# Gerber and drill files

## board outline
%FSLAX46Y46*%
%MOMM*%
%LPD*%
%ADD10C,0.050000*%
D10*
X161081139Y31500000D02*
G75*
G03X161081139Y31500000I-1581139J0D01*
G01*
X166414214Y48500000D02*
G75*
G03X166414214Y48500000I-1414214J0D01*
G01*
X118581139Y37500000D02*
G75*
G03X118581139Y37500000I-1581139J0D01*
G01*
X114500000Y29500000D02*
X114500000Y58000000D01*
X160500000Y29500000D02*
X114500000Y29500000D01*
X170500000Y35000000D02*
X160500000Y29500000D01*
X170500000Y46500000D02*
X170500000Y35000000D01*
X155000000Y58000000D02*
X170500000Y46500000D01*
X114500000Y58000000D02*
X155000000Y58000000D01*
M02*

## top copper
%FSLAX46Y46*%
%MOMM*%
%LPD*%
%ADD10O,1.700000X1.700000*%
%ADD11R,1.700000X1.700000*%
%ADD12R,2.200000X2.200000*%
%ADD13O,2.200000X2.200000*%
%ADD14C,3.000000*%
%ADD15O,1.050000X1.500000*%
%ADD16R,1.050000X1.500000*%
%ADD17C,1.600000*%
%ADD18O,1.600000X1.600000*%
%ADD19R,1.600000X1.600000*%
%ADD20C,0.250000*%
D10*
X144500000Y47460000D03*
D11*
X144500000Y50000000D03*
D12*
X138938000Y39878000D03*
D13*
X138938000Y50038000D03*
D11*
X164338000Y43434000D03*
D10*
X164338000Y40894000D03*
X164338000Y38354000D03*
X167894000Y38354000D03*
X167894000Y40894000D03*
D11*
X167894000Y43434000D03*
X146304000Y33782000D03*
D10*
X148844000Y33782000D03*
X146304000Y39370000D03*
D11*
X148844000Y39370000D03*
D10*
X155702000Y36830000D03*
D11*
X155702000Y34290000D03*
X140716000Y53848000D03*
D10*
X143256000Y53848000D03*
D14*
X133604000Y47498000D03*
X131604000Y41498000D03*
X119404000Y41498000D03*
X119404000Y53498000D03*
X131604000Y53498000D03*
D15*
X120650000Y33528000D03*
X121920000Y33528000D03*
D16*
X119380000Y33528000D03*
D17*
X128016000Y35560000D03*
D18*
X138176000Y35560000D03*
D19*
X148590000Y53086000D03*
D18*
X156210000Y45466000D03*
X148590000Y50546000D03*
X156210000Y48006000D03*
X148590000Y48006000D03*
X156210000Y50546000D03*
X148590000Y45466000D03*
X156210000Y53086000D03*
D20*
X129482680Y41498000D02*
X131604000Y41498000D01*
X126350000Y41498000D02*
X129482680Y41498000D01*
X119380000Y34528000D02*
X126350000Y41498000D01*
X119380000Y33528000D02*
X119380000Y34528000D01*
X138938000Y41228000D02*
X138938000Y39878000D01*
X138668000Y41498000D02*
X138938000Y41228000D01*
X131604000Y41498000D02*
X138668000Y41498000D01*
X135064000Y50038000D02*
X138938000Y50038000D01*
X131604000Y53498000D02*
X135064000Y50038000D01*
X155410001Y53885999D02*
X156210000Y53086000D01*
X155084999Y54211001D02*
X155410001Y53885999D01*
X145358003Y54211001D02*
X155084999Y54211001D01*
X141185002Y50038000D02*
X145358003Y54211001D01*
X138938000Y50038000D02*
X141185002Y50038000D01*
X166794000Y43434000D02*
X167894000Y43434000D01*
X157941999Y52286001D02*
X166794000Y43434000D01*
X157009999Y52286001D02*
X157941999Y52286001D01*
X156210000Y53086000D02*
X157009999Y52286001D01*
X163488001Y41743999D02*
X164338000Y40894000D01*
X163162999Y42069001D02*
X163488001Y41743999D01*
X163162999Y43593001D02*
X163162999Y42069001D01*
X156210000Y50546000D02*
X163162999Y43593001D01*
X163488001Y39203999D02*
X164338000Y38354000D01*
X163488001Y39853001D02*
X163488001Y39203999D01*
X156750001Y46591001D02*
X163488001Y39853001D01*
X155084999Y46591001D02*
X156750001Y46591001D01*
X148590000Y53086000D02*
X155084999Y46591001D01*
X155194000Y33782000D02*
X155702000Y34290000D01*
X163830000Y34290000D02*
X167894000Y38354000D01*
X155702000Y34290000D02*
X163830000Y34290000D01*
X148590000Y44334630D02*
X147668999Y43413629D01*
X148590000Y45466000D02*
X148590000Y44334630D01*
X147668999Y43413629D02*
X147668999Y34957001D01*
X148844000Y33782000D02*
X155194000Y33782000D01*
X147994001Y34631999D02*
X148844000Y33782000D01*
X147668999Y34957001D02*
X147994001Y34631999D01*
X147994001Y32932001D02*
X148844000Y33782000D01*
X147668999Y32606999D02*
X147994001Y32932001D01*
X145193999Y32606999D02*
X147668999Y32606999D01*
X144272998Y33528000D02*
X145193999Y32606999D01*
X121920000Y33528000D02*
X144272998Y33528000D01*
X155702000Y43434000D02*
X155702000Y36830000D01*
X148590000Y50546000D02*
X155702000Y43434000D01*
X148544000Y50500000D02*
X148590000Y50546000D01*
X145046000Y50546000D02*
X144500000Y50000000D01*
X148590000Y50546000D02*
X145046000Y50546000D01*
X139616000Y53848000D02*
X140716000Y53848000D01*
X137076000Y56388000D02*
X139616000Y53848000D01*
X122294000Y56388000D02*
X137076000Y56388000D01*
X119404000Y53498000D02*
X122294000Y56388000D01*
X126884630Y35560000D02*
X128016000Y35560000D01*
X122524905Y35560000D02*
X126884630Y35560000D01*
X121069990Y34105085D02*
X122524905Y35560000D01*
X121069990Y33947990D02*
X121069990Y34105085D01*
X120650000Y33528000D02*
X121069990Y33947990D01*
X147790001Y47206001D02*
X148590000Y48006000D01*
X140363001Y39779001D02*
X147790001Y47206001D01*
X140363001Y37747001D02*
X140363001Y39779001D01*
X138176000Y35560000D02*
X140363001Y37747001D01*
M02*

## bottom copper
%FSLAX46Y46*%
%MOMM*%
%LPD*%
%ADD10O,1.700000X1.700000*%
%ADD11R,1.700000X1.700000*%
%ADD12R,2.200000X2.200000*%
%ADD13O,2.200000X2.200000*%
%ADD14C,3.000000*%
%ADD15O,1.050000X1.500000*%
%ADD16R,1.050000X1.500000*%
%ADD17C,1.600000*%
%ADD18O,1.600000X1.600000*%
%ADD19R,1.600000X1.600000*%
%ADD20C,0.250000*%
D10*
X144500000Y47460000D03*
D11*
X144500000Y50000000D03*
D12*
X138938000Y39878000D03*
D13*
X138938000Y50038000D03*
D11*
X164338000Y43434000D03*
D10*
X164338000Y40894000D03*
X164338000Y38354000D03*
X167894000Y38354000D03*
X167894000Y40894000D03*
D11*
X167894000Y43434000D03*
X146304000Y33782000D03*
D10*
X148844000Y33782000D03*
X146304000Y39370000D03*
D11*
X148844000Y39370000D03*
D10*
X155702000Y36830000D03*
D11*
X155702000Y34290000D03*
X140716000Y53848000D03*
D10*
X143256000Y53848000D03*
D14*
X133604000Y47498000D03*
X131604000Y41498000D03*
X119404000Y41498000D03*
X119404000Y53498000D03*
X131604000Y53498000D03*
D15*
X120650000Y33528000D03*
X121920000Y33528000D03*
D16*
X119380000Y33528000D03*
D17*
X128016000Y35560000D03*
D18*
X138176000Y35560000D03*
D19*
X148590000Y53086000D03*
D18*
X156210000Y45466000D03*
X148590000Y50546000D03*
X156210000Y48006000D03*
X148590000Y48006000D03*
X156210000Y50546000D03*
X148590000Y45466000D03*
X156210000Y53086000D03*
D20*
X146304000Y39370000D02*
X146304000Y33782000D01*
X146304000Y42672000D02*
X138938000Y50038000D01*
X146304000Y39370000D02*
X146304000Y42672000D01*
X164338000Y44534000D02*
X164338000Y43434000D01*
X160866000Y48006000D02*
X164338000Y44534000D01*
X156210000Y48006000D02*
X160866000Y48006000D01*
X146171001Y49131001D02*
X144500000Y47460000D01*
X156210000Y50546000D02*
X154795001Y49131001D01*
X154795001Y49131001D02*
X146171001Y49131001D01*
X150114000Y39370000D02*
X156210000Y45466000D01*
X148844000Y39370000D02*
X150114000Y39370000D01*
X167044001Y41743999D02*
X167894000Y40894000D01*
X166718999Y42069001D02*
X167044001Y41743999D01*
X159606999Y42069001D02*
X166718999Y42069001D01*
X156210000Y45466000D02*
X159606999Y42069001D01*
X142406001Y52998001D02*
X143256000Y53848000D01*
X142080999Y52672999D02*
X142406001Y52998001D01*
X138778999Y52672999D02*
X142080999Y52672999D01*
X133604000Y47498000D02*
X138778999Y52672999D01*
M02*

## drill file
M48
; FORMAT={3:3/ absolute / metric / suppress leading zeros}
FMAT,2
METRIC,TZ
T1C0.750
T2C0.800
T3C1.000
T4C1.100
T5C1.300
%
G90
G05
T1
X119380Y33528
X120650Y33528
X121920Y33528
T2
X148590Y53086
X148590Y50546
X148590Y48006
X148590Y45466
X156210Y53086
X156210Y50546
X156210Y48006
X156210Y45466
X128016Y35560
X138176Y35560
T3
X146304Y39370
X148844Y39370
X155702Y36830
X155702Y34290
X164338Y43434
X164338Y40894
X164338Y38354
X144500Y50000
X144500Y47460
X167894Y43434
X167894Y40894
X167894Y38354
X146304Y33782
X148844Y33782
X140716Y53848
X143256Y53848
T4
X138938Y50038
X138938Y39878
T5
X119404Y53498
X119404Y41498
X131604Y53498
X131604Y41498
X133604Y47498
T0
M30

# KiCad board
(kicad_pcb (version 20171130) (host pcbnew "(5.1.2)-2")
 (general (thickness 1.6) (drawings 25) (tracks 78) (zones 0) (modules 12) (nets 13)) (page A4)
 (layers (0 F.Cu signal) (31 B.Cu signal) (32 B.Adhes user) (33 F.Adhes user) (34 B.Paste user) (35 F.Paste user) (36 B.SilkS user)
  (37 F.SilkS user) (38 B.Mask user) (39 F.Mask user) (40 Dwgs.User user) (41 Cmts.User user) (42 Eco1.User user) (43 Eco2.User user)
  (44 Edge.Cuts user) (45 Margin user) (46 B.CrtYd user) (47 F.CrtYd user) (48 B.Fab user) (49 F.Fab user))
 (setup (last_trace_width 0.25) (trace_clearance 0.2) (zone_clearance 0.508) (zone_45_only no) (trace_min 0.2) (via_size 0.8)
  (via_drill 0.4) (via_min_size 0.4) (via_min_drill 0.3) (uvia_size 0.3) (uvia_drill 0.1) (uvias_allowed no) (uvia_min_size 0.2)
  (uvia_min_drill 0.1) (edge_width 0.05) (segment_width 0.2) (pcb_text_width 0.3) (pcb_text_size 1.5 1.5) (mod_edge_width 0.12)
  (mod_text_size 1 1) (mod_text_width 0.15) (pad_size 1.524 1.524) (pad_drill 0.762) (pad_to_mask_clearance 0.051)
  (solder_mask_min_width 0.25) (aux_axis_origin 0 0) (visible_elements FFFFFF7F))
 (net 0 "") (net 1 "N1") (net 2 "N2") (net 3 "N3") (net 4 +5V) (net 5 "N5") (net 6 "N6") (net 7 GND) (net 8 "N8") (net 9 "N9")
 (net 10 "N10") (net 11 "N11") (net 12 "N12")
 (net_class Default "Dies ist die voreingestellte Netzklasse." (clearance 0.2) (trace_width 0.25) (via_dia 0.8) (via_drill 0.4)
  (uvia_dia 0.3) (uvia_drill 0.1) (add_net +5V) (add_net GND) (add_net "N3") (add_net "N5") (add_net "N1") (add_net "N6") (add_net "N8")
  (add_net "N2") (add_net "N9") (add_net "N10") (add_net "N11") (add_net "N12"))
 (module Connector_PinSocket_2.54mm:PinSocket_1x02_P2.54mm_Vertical (layer F.Cu) (at 144.5 -50)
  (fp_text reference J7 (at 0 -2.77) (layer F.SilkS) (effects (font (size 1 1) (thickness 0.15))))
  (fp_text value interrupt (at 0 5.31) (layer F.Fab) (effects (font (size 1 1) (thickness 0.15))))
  (pad 2 thru_hole oval (at 0 2.54) (size 1.7 1.7) (drill 1) (layers *.Cu *.Mask) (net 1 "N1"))
  (pad 1 thru_hole rect (at 0 0) (size 1.7 1.7) (drill 1) (layers *.Cu *.Mask) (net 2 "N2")))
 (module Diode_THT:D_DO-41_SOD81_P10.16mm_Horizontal (layer F.Cu) (at 138.938 -39.878 90)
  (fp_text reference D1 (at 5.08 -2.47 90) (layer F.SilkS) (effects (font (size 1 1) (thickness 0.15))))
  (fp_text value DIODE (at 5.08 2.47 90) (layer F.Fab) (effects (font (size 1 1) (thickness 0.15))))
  (pad 1 thru_hole rect (at 0 0 90) (size 2.2 2.2) (drill 1.1) (layers *.Cu *.Mask) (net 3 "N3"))
  (pad 2 thru_hole oval (at 10.16 0 90) (size 2.2 2.2) (drill 1.1) (layers *.Cu *.Mask) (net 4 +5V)))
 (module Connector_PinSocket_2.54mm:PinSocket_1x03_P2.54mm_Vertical (layer F.Cu) (at 164.338 -43.434)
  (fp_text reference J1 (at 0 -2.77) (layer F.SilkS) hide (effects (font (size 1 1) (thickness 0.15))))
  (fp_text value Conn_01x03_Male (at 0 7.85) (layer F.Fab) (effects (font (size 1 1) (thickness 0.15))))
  (pad 1 thru_hole rect (at 0 0) (size 1.7 1.7) (drill 1) (layers *.Cu *.Mask) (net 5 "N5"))
  (pad 2 thru_hole oval (at 0 2.54) (size 1.7 1.7) (drill 1) (layers *.Cu *.Mask) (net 1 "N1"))
  (pad 3 thru_hole oval (at 0 5.08) (size 1.7 1.7) (drill 1) (layers *.Cu *.Mask) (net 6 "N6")))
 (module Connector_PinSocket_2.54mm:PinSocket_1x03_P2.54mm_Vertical (layer F.Cu) (at 167.894 -43.434)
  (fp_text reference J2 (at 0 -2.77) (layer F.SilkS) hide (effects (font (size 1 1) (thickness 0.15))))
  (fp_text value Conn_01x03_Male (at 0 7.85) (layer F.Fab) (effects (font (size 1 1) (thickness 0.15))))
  (pad 3 thru_hole oval (at 0 5.08) (size 1.7 1.7) (drill 1) (layers *.Cu *.Mask) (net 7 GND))
  (pad 2 thru_hole oval (at 0 2.54) (size 1.7 1.7) (drill 1) (layers *.Cu *.Mask) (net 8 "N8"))
  (pad 1 thru_hole rect (at 0 0) (size 1.7 1.7) (drill 1) (layers *.Cu *.Mask) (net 4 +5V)))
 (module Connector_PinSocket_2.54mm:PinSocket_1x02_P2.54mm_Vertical (layer F.Cu) (at 146.304 -33.782 90)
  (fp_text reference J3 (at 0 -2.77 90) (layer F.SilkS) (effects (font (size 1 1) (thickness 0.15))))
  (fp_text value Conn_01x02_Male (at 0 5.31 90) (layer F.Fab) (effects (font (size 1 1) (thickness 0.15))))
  (pad 1 thru_hole rect (at 0 0 90) (size 1.7 1.7) (drill 1) (layers *.Cu *.Mask) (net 4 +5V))
  (pad 2 thru_hole oval (at 0 2.54 90) (size 1.7 1.7) (drill 1) (layers *.Cu *.Mask) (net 7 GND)))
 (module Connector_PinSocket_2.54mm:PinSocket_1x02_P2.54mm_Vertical (layer F.Cu) (at 148.844 -39.37 270)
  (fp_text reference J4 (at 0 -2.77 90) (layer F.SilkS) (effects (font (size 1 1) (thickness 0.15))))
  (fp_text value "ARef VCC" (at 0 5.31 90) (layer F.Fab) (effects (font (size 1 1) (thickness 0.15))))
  (pad 2 thru_hole oval (at 0 2.54 270) (size 1.7 1.7) (drill 1) (layers *.Cu *.Mask) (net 4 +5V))
  (pad 1 thru_hole rect (at 0 0 270) (size 1.7 1.7) (drill 1) (layers *.Cu *.Mask) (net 8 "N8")))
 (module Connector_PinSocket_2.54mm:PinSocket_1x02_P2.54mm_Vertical (layer F.Cu) (at 155.702 -34.29 180)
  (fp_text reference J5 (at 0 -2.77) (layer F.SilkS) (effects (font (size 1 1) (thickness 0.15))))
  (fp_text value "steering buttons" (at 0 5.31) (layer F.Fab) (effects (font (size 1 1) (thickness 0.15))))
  (pad 2 thru_hole oval (at 0 2.54 180) (size 1.7 1.7) (drill 1) (layers *.Cu *.Mask) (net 2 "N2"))
  (pad 1 thru_hole rect (at 0 0 180) (size 1.7 1.7) (drill 1) (layers *.Cu *.Mask) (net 7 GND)))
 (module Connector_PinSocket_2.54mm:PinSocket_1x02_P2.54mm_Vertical (layer F.Cu) (at 140.716 -53.848 90)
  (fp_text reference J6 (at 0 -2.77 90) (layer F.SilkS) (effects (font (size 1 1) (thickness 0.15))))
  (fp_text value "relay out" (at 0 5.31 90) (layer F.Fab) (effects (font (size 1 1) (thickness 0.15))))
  (pad 1 thru_hole rect (at 0 0 90) (size 1.7 1.7) (drill 1) (layers *.Cu *.Mask) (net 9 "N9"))
  (pad 2 thru_hole oval (at 0 2.54 90) (size 1.7 1.7) (drill 1) (layers *.Cu *.Mask) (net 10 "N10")))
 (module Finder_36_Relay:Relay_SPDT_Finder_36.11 (layer F.Cu) (at 133.604 -47.498 180)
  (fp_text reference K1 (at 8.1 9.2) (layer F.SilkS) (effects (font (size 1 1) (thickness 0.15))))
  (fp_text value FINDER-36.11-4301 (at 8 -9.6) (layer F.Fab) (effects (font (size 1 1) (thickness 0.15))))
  (pad 11 thru_hole circle (at 0 0 180) (size 3 3) (drill 1.3) (layers *.Cu *.Mask) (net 10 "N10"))
  (pad A2 thru_hole circle (at 2 -6 180) (size 3 3) (drill 1.3) (layers *.Cu *.Mask) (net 3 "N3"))
  (pad 12 thru_hole circle (at 14.2 -6 180) (size 3 3) (drill 1.3) (layers *.Cu *.Mask))
  (pad 14 thru_hole circle (at 14.2 6 180) (size 3 3) (drill 1.3) (layers *.Cu *.Mask) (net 9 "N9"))
  (pad A1 thru_hole circle (at 2 6 180) (size 3 3) (drill 1.3) (layers *.Cu *.Mask) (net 4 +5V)))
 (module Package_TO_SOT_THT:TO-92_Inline (layer F.Cu) (at 119.38 -33.528)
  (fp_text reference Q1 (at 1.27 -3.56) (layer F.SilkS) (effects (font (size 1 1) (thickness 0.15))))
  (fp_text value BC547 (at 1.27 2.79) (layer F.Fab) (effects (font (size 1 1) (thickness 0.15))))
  (pad 2 thru_hole oval (at 1.27 0) (size 1.05 1.5) (drill 0.75) (layers *.Cu *.Mask) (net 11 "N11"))
  (pad 3 thru_hole oval (at 2.54 0) (size 1.05 1.5) (drill 0.75) (layers *.Cu *.Mask) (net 7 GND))
  (pad 1 thru_hole rect (at 0 0) (size 1.05 1.5) (drill 0.75) (layers *.Cu *.Mask) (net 3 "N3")))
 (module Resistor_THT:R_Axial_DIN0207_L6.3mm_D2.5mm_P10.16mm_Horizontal (layer F.Cu) (at 128.016 -35.56)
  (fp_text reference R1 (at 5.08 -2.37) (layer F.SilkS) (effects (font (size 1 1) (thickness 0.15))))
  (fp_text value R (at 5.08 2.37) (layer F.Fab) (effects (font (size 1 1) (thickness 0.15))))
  (pad 1 thru_hole circle (at 0 0) (size 1.6 1.6) (drill 0.8) (layers *.Cu *.Mask) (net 11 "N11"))
  (pad 2 thru_hole oval (at 10.16 0) (size 1.6 1.6) (drill 0.8) (layers *.Cu *.Mask) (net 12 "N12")))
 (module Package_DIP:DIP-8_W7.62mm (layer F.Cu) (at 148.59 -53.086)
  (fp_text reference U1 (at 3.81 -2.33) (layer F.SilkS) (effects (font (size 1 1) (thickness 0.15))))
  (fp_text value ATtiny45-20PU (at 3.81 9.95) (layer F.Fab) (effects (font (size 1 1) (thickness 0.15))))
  (pad 1 thru_hole rect (at 0 0) (size 1.6 1.6) (drill 0.8) (layers *.Cu *.Mask) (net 6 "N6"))
  (pad 5 thru_hole oval (at 7.62 7.62) (size 1.6 1.6) (drill 0.8) (layers *.Cu *.Mask) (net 8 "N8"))
  (pad 2 thru_hole oval (at 0 2.54) (size 1.6 1.6) (drill 0.8) (layers *.Cu *.Mask) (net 2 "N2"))
  (pad 6 thru_hole oval (at 7.62 5.08) (size 1.6 1.6) (drill 0.8) (layers *.Cu *.Mask) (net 5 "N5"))
  (pad 3 thru_hole oval (at 0 5.08) (size 1.6 1.6) (drill 0.8) (layers *.Cu *.Mask) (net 12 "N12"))
  (pad 7 thru_hole oval (at 7.62 2.54) (size 1.6 1.6) (drill 0.8) (layers *.Cu *.Mask) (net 1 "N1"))
  (pad 4 thru_hole oval (at 0 7.62) (size 1.6 1.6) (drill 0.8) (layers *.Cu *.Mask) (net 7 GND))
  (pad 8 thru_hole oval (at 7.62 0) (size 1.6 1.6) (drill 0.8) (layers *.Cu *.Mask) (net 4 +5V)))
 (gr_circle (center 159.5 -31.5) (end 160 -33) (layer Edge.Cuts) (width 0.05))
 (gr_circle (center 165 -48.5) (end 166 -47.5) (layer Edge.Cuts) (width 0.05))
 (gr_circle (center 117 -37.5) (end 115.5 -38) (layer Edge.Cuts) (width 0.05))
 (gr_line (start 114.5 -29.5) (end 114.5 -58) (layer Edge.Cuts) (width 0.05))
 (gr_line (start 160.5 -29.5) (end 114.5 -29.5) (layer Edge.Cuts) (width 0.05))
 (gr_line (start 170.5 -35) (end 160.5 -29.5) (layer Edge.Cuts) (width 0.05))
 (gr_line (start 170.5 -46.5) (end 170.5 -35) (layer Edge.Cuts) (width 0.05))
 (gr_line (start 155 -58) (end 170.5 -46.5) (layer Edge.Cuts) (width 0.05))
 (gr_line (start 114.5 -58) (end 155 -58) (layer Edge.Cuts) (width 0.05))
 (segment (start 129.48268 -41.498) (end 131.604 -41.498) (width 0.25) (layer F.Cu) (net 3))
 (segment (start 126.35 -41.498) (end 129.48268 -41.498) (width 0.25) (layer F.Cu) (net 3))
 (segment (start 119.38 -34.528) (end 126.35 -41.498) (width 0.25) (layer F.Cu) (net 3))
 (segment (start 119.38 -33.528) (end 119.38 -34.528) (width 0.25) (layer F.Cu) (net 3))
 (segment (start 138.938 -41.228) (end 138.938 -39.878) (width 0.25) (layer F.Cu) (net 3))
 (segment (start 138.668 -41.498) (end 138.938 -41.228) (width 0.25) (layer F.Cu) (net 3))
 (segment (start 131.604 -41.498) (end 138.668 -41.498) (width 0.25) (layer F.Cu) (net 3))
 (segment (start 135.064 -50.038) (end 138.938 -50.038) (width 0.25) (layer F.Cu) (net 4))
 (segment (start 131.604 -53.498) (end 135.064 -50.038) (width 0.25) (layer F.Cu) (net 4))
 (segment (start 155.410001 -53.885999) (end 156.21 -53.086) (width 0.25) (layer F.Cu) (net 4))
 (segment (start 155.084999 -54.211001) (end 155.410001 -53.885999) (width 0.25) (layer F.Cu) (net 4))
 (segment (start 145.358003 -54.211001) (end 155.084999 -54.211001) (width 0.25) (layer F.Cu) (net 4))
 (segment (start 141.185002 -50.038) (end 145.358003 -54.211001) (width 0.25) (layer F.Cu) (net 4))
 (segment (start 138.938 -50.038) (end 141.185002 -50.038) (width 0.25) (layer F.Cu) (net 4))
 (segment (start 146.304 -39.37) (end 146.304 -33.782) (width 0.25) (layer B.Cu) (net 4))
 (segment (start 166.794 -43.434) (end 167.894 -43.434) (width 0.25) (layer F.Cu) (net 4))
 (segment (start 157.941999 -52.286001) (end 166.794 -43.434) (width 0.25) (layer F.Cu) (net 4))
 (segment (start 157.009999 -52.286001) (end 157.941999 -52.286001) (width 0.25) (layer F.Cu) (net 4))
 (segment (start 156.21 -53.086) (end 157.009999 -52.286001) (width 0.25) (layer F.Cu) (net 4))
 (segment (start 146.304 -42.672) (end 138.938 -50.038) (width 0.25) (layer B.Cu) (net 4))
 (segment (start 146.304 -39.37) (end 146.304 -42.672) (width 0.25) (layer B.Cu) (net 4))
 (segment (start 164.338 -44.534) (end 164.338 -43.434) (width 0.25) (layer B.Cu) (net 5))
 (segment (start 160.866 -48.006) (end 164.338 -44.534) (width 0.25) (layer B.Cu) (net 5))
 (segment (start 156.21 -48.006) (end 160.866 -48.006) (width 0.25) (layer B.Cu) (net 5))
 (segment (start 163.488001 -41.743999) (end 164.338 -40.894) (width 0.25) (layer F.Cu) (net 1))
 (segment (start 163.162999 -42.069001) (end 163.488001 -41.743999) (width 0.25) (layer F.Cu) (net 1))
 (segment (start 163.162999 -43.593001) (end 163.162999 -42.069001) (width 0.25) (layer F.Cu) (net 1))
 (segment (start 156.21 -50.546) (end 163.162999 -43.593001) (width 0.25) (layer F.Cu) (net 1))
 (segment (start 146.171001 -49.131001) (end 144.5 -47.46) (width 0.25) (layer B.Cu) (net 1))
 (segment (start 156.21 -50.546) (end 154.795001 -49.131001) (width 0.25) (layer B.Cu) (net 1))
 (segment (start 154.795001 -49.131001) (end 146.171001 -49.131001) (width 0.25) (layer B.Cu) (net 1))
 (segment (start 163.488001 -39.203999) (end 164.338 -38.354) (width 0.25) (layer F.Cu) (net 6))
 (segment (start 163.488001 -39.853001) (end 163.488001 -39.203999) (width 0.25) (layer F.Cu) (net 6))
 (segment (start 156.750001 -46.591001) (end 163.488001 -39.853001) (width 0.25) (layer F.Cu) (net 6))
 (segment (start 155.084999 -46.591001) (end 156.750001 -46.591001) (width 0.25) (layer F.Cu) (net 6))
 (segment (start 148.59 -53.086) (end 155.084999 -46.591001) (width 0.25) (layer F.Cu) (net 6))
 (segment (start 155.194 -33.782) (end 155.702 -34.29) (width 0.25) (layer F.Cu) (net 7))
 (segment (start 163.83 -34.29) (end 167.894 -38.354) (width 0.25) (layer F.Cu) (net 7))
 (segment (start 155.702 -34.29) (end 163.83 -34.29) (width 0.25) (layer F.Cu) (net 7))
 (segment (start 148.59 -44.33463) (end 147.668999 -43.413629) (width 0.25) (layer F.Cu) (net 7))
 (segment (start 148.59 -45.466) (end 148.59 -44.33463) (width 0.25) (layer F.Cu) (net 7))
 (segment (start 147.668999 -43.413629) (end 147.668999 -34.957001) (width 0.25) (layer F.Cu) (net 7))
 (segment (start 148.844 -33.782) (end 155.194 -33.782) (width 0.25) (layer F.Cu) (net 7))
 (segment (start 147.994001 -34.631999) (end 148.844 -33.782) (width 0.25) (layer F.Cu) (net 7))
 (segment (start 147.668999 -34.957001) (end 147.994001 -34.631999) (width 0.25) (layer F.Cu) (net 7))
 (segment (start 147.994001 -32.932001) (end 148.844 -33.782) (width 0.25) (layer F.Cu) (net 7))
 (segment (start 147.668999 -32.606999) (end 147.994001 -32.932001) (width 0.25) (layer F.Cu) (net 7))
 (segment (start 145.193999 -32.606999) (end 147.668999 -32.606999) (width 0.25) (layer F.Cu) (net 7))
 (segment (start 144.272998 -33.528) (end 145.193999 -32.606999) (width 0.25) (layer F.Cu) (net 7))
 (segment (start 121.92 -33.528) (end 144.272998 -33.528) (width 0.25) (layer F.Cu) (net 7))
 (segment (start 150.114 -39.37) (end 156.21 -45.466) (width 0.25) (layer B.Cu) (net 8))
 (segment (start 148.844 -39.37) (end 150.114 -39.37) (width 0.25) (layer B.Cu) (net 8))
 (segment (start 167.044001 -41.743999) (end 167.894 -40.894) (width 0.25) (layer B.Cu) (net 8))
 (segment (start 166.718999 -42.069001) (end 167.044001 -41.743999) (width 0.25) (layer B.Cu) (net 8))
 (segment (start 159.606999 -42.069001) (end 166.718999 -42.069001) (width 0.25) (layer B.Cu) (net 8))
 (segment (start 156.21 -45.466) (end 159.606999 -42.069001) (width 0.25) (layer B.Cu) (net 8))
 (segment (start 155.702 -43.434) (end 155.702 -36.83) (width 0.25) (layer F.Cu) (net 2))
 (segment (start 148.59 -50.546) (end 155.702 -43.434) (width 0.25) (layer F.Cu) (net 2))
 (segment (start 148.544 -50.5) (end 148.59 -50.546) (width 0.25) (layer F.Cu) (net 2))
 (segment (start 145.046 -50.546) (end 144.5 -50) (width 0.25) (layer F.Cu) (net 2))
 (segment (start 148.59 -50.546) (end 145.046 -50.546) (width 0.25) (layer F.Cu) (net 2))
 (segment (start 139.616 -53.848) (end 140.716 -53.848) (width 0.25) (layer F.Cu) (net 9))
 (segment (start 137.076 -56.388) (end 139.616 -53.848) (width 0.25) (layer F.Cu) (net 9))
 (segment (start 122.294 -56.388) (end 137.076 -56.388) (width 0.25) (layer F.Cu) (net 9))
 (segment (start 119.404 -53.498) (end 122.294 -56.388) (width 0.25) (layer F.Cu) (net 9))
 (segment (start 142.406001 -52.998001) (end 143.256 -53.848) (width 0.25) (layer B.Cu) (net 10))
 (segment (start 142.080999 -52.672999) (end 142.406001 -52.998001) (width 0.25) (layer B.Cu) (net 10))
 (segment (start 138.778999 -52.672999) (end 142.080999 -52.672999) (width 0.25) (layer B.Cu) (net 10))
 (segment (start 133.604 -47.498) (end 138.778999 -52.672999) (width 0.25) (layer B.Cu) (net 10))
 (segment (start 126.88463 -35.56) (end 128.016 -35.56) (width 0.25) (layer F.Cu) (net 11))
 (segment (start 122.524905 -35.56) (end 126.88463 -35.56) (width 0.25) (layer F.Cu) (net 11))
 (segment (start 121.06999 -34.105085) (end 122.524905 -35.56) (width 0.25) (layer F.Cu) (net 11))
 (segment (start 121.06999 -33.94799) (end 121.06999 -34.105085) (width 0.25) (layer F.Cu) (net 11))
 (segment (start 120.65 -33.528) (end 121.06999 -33.94799) (width 0.25) (layer F.Cu) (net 11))
 (segment (start 147.790001 -47.206001) (end 148.59 -48.006) (width 0.25) (layer F.Cu) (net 12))
 (segment (start 140.363001 -39.779001) (end 147.790001 -47.206001) (width 0.25) (layer F.Cu) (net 12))
 (segment (start 140.363001 -37.747001) (end 140.363001 -39.779001) (width 0.25) (layer F.Cu) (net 12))
 (segment (start 138.176 -35.56) (end 140.363001 -37.747001) (width 0.25) (layer F.Cu) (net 12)))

